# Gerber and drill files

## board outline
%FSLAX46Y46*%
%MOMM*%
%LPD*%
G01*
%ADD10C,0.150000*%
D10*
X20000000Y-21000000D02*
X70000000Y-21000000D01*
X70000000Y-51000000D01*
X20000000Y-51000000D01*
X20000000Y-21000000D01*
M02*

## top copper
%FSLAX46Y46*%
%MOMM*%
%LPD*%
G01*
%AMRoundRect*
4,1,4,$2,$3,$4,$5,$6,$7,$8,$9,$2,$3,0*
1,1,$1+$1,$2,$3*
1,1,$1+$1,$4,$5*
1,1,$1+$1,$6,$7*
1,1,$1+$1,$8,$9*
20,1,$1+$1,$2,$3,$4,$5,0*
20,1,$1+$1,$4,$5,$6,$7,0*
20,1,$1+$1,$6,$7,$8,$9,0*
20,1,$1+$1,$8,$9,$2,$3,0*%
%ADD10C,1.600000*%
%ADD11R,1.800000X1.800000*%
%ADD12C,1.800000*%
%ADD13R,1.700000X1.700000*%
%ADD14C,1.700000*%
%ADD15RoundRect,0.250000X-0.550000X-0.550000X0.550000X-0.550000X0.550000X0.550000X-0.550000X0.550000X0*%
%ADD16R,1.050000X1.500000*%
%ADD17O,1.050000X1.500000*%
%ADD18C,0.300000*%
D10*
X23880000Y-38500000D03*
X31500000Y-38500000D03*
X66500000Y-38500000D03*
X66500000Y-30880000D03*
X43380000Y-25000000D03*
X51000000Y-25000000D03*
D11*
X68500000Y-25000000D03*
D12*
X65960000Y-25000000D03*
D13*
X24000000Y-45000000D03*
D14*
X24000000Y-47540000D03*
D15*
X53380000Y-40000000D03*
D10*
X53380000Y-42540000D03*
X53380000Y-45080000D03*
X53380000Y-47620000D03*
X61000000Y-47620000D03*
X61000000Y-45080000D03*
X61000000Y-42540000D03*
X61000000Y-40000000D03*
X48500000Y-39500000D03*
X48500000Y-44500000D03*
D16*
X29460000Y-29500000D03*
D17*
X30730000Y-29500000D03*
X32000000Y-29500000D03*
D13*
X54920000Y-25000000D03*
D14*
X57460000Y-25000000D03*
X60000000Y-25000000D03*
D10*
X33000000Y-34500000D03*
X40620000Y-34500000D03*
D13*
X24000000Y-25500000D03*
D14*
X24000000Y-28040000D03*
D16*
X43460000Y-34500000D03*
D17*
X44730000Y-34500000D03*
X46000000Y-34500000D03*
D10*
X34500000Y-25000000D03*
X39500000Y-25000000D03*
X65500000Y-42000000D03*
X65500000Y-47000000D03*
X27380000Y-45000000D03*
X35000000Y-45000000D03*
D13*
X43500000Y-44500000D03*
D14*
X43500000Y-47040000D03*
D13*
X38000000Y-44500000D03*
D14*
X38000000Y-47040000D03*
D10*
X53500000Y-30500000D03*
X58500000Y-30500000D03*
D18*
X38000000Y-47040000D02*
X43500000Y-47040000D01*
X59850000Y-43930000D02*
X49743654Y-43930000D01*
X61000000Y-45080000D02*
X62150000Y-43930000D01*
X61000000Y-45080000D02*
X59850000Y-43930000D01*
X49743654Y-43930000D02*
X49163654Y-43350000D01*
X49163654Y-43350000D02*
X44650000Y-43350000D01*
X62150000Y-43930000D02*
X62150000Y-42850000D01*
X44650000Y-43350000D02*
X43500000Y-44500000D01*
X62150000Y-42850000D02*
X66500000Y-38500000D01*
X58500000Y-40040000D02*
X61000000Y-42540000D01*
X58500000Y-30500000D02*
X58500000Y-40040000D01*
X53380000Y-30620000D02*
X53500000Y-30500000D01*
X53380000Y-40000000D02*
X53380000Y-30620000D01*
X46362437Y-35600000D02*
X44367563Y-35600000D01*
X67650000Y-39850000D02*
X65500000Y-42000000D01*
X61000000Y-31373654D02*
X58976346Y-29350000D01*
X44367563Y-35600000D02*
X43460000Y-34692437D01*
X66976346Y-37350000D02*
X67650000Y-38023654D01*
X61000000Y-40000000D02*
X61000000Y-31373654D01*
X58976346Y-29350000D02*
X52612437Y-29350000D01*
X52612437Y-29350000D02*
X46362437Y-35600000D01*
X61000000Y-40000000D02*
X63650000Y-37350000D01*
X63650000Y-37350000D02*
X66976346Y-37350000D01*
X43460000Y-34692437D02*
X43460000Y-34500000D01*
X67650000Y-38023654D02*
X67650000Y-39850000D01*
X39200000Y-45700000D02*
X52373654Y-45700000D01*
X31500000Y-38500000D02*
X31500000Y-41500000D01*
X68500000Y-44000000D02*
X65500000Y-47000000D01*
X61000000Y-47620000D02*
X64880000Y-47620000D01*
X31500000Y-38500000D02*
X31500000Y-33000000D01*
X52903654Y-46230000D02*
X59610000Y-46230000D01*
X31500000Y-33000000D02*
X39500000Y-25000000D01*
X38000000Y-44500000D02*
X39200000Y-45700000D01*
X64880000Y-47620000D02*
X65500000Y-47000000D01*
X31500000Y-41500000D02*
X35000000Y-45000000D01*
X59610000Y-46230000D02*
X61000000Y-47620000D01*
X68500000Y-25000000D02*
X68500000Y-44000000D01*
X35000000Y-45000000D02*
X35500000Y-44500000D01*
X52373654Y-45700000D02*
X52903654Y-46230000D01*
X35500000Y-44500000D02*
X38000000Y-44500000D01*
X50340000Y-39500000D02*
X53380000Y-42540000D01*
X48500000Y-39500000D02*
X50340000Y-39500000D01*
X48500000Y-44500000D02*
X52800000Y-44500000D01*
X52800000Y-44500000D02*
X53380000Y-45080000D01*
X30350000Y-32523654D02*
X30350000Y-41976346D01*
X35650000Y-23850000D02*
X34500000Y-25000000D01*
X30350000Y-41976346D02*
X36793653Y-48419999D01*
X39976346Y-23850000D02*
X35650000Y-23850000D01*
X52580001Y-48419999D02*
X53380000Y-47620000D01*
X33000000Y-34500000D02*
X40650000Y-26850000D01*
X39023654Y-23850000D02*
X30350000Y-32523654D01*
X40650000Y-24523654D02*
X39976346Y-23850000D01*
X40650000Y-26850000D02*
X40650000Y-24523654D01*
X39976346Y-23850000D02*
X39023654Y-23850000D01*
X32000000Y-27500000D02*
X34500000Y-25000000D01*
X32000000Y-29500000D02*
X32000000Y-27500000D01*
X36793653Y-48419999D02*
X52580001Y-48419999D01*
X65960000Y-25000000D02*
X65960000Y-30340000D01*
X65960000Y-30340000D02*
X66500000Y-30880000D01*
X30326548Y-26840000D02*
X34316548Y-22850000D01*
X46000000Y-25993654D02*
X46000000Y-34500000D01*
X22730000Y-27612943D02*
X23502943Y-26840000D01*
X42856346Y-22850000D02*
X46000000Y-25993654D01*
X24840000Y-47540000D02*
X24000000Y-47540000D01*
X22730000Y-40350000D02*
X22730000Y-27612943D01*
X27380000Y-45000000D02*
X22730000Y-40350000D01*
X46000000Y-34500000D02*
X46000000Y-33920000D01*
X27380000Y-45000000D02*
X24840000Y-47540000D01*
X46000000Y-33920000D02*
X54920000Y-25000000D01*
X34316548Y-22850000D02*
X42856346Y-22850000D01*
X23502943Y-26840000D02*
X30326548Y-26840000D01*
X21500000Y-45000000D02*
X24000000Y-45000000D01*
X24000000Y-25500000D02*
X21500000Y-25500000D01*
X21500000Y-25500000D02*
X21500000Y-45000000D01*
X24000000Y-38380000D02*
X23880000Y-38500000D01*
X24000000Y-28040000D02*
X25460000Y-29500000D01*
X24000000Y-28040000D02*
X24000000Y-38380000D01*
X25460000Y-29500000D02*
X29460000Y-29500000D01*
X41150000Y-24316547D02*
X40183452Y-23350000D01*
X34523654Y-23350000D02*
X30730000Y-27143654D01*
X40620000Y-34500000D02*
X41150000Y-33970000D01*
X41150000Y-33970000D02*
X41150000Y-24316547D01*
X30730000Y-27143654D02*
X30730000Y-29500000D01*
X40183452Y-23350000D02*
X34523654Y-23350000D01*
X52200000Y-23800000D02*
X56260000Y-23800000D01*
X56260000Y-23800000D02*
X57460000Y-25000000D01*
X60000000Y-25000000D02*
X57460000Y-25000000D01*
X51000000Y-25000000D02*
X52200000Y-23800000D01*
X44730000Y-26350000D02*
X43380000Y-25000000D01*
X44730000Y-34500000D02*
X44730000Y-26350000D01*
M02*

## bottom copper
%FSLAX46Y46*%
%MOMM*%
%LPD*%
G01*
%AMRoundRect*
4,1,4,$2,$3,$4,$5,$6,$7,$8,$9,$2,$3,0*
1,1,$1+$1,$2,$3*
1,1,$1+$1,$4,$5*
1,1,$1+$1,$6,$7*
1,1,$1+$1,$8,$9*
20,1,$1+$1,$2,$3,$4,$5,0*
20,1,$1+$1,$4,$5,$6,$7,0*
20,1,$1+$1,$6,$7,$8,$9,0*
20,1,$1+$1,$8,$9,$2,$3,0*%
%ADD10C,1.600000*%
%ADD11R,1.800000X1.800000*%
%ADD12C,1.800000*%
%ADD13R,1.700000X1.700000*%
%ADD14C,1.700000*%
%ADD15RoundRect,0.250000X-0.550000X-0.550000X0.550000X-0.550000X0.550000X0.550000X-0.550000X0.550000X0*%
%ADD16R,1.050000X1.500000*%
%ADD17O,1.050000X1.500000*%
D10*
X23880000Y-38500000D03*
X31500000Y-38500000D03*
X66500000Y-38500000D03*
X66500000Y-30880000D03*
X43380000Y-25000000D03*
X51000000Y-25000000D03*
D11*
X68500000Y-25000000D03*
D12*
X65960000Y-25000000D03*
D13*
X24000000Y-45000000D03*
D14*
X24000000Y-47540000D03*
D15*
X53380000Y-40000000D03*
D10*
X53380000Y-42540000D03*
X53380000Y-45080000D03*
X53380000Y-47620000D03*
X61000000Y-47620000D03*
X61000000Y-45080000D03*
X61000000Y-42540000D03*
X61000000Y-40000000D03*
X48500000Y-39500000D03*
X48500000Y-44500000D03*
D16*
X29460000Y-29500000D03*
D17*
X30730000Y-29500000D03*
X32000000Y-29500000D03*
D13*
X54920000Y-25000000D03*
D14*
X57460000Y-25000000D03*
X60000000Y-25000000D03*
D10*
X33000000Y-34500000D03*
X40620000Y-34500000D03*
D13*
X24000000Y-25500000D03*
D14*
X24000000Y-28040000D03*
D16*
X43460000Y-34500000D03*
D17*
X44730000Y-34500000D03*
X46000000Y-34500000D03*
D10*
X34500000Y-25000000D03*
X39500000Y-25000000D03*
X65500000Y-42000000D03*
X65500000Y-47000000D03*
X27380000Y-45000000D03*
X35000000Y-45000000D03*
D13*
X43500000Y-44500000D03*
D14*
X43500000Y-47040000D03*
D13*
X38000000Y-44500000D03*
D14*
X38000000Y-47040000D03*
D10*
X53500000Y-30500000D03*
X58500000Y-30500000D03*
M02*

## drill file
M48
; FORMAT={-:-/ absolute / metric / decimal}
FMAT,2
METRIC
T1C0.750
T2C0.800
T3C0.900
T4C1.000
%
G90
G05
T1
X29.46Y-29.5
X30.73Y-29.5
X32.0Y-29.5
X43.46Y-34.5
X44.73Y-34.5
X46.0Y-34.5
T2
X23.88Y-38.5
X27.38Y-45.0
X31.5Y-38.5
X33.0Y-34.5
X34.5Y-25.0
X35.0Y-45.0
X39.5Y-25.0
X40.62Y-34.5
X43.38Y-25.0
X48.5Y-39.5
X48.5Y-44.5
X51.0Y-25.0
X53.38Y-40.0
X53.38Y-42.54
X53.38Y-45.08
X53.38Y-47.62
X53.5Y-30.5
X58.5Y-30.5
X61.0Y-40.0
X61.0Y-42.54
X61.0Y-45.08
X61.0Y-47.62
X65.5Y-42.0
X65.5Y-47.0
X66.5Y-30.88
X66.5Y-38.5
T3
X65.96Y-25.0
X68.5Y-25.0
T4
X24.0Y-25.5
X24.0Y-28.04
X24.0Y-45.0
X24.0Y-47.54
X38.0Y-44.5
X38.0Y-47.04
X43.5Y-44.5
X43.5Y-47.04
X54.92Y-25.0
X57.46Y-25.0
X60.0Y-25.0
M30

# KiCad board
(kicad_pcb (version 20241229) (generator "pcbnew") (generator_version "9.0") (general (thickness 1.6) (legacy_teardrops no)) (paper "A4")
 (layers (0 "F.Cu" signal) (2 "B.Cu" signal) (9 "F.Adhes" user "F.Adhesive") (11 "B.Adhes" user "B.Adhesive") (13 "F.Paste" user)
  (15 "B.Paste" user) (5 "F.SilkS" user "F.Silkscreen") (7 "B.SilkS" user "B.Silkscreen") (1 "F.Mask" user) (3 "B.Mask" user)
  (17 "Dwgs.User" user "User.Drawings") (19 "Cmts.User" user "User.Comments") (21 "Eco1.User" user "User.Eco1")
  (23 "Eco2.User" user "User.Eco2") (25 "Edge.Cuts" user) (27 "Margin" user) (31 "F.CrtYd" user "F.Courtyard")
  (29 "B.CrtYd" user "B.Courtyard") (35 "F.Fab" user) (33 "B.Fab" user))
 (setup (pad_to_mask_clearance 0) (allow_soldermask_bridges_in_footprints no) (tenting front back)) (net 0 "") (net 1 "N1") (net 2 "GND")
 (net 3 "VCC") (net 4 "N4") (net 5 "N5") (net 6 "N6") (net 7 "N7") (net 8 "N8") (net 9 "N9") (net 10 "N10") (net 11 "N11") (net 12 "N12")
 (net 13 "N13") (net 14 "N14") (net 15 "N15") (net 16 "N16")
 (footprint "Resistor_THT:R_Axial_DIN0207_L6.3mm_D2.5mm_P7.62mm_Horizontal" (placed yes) (layer "F.Cu") (at 23.88 38.5)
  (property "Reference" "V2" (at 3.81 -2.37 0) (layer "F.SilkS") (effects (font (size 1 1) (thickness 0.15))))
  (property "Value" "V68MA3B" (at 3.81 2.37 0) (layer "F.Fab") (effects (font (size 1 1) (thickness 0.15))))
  (pad "1" thru_hole circle (at 0 0) (size 1.6 1.6) (drill 0.8) (layers "*.Cu" "*.Mask") (remove_unused_layers no) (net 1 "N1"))
  (pad "2" thru_hole circle (at 7.62 0) (size 1.6 1.6) (drill 0.8) (layers "*.Cu" "*.Mask") (remove_unused_layers no) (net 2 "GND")))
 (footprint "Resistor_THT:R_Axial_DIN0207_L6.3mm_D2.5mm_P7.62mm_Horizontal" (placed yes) (layer "F.Cu") (at 66.5 38.5 90)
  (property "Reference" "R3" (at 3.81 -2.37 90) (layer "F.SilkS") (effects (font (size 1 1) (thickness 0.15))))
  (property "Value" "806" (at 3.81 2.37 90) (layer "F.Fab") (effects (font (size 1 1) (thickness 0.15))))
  (pad "1" thru_hole circle (at 0 0 90) (size 1.6 1.6) (drill 0.8) (layers "*.Cu" "*.Mask") (remove_unused_layers no) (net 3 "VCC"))
  (pad "2" thru_hole circle (at 7.62 0 90) (size 1.6 1.6) (drill 0.8) (layers "*.Cu" "*.Mask") (remove_unused_layers no) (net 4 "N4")))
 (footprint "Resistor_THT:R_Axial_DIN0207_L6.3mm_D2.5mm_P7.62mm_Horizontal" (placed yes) (layer "F.Cu") (at 43.38 25)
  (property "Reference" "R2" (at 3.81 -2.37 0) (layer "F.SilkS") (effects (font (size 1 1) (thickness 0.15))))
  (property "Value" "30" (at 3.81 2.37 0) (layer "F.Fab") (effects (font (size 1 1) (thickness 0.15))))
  (pad "1" thru_hole circle (at 0 0) (size 1.6 1.6) (drill 0.8) (layers "*.Cu" "*.Mask") (remove_unused_layers no) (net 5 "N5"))
  (pad "2" thru_hole circle (at 7.62 0) (size 1.6 1.6) (drill 0.8) (layers "*.Cu" "*.Mask") (remove_unused_layers no) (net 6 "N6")))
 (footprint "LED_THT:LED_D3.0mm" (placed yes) (layer "F.Cu") (at 68.5 25 180)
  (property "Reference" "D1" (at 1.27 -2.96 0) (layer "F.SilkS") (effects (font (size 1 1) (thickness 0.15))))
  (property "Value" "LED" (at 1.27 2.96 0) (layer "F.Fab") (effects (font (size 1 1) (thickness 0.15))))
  (pad "1" thru_hole rect (at 0 0 180) (size 1.8 1.8) (drill 0.9) (layers "*.Cu" "*.Mask") (remove_unused_layers no) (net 2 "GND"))
  (pad "2" thru_hole circle (at 2.54 0 180) (size 1.8 1.8) (drill 0.9) (layers "*.Cu" "*.Mask") (remove_unused_layers no) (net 4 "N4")))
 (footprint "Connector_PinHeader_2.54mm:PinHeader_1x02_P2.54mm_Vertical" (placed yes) (layer "F.Cu") (at 24 45)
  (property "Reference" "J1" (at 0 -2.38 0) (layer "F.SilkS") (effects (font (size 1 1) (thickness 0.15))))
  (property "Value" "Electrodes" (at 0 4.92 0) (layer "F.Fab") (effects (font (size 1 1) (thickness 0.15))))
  (pad "1" thru_hole rect (at 0 0) (size 1.7 1.7) (drill 1) (layers "*.Cu" "*.Mask") (remove_unused_layers no) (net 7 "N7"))
  (pad "2" thru_hole circle (at 0 2.54) (size 1.7 1.7) (drill 1) (layers "*.Cu" "*.Mask") (remove_unused_layers no) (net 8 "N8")))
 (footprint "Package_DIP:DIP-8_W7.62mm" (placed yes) (layer "F.Cu") (at 53.38 40)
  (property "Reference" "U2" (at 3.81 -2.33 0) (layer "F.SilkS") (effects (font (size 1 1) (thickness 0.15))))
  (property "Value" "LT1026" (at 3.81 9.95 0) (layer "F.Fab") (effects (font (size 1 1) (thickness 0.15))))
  (pad "1" thru_hole roundrect (at 0 0) (size 1.6 1.6) (drill 0.8) (layers "*.Cu" "*.Mask") (remove_unused_layers no)
   (roundrect_rratio 0.15625) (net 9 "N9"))
  (pad "2" thru_hole circle (at 0 2.54) (size 1.6 1.6) (drill 0.8) (layers "*.Cu" "*.Mask") (remove_unused_layers no) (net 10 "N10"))
  (pad "3" thru_hole circle (at 0 5.08) (size 1.6 1.6) (drill 0.8) (layers "*.Cu" "*.Mask") (remove_unused_layers no) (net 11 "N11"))
  (pad "4" thru_hole circle (at 0 7.62) (size 1.6 1.6) (drill 0.8) (layers "*.Cu" "*.Mask") (remove_unused_layers no) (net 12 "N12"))
  (pad "5" thru_hole circle (at 7.62 7.62) (size 1.6 1.6) (drill 0.8) (layers "*.Cu" "*.Mask") (remove_unused_layers no) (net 2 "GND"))
  (pad "6" thru_hole circle (at 7.62 5.08) (size 1.6 1.6) (drill 0.8) (layers "*.Cu" "*.Mask") (remove_unused_layers no) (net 3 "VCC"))
  (pad "7" thru_hole circle (at 7.62 2.54) (size 1.6 1.6) (drill 0.8) (layers "*.Cu" "*.Mask") (remove_unused_layers no) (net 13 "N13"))
  (pad "8" thru_hole circle (at 7.62 0) (size 1.6 1.6) (drill 0.8) (layers "*.Cu" "*.Mask") (remove_unused_layers no) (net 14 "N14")))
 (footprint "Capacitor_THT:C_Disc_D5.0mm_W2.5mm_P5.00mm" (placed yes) (layer "F.Cu") (at 48.5 39.5 -90)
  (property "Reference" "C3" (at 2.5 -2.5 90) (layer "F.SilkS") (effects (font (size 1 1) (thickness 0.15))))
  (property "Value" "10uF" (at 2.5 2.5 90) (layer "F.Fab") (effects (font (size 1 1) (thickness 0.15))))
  (pad "1" thru_hole circle (at 0 0 270) (size 1.6 1.6) (drill 0.8) (layers "*.Cu" "*.Mask") (remove_unused_layers no) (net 10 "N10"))
  (pad "2" thru_hole circle (at 5 0 270) (size 1.6 1.6) (drill 0.8) (layers "*.Cu" "*.Mask") (remove_unused_layers no) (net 11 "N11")))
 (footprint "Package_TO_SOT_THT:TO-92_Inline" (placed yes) (layer "F.Cu") (at 29.46 29.5)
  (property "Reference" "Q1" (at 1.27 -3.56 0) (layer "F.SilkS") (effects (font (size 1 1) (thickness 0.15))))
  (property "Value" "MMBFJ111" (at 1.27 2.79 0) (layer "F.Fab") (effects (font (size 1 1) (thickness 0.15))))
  (pad "1" thru_hole rect (at 0 0) (size 1.05 1.5) (drill 0.75) (layers "*.Cu" "*.Mask") (remove_unused_layers no) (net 1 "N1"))
  (pad "2" thru_hole oval (at 1.27 0) (size 1.05 1.5) (drill 0.75) (layers "*.Cu" "*.Mask") (remove_unused_layers no) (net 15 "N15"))
  (pad "3" thru_hole oval (at 2.54 0) (size 1.05 1.5) (drill 0.75) (layers "*.Cu" "*.Mask") (remove_unused_layers no) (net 12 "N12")))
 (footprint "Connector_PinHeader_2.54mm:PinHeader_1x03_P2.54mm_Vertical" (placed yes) (layer "F.Cu") (at 54.92 25 90)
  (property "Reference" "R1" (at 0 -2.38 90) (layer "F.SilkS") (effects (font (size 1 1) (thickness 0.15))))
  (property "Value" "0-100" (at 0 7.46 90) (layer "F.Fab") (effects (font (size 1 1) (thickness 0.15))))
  (pad "1" thru_hole rect (at 0 0 90) (size 1.7 1.7) (drill 1) (layers "*.Cu" "*.Mask") (remove_unused_layers no) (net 8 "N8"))
  (pad "2" thru_hole circle (at 0 2.54 90) (size 1.7 1.7) (drill 1) (layers "*.Cu" "*.Mask") (remove_unused_layers no) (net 6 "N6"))
  (pad "3" thru_hole circle (at 0 5.08 90) (size 1.7 1.7) (drill 1) (layers "*.Cu" "*.Mask") (remove_unused_layers no) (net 6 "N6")))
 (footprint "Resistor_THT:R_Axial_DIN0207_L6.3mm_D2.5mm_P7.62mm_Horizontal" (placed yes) (layer "F.Cu") (at 33 34.5)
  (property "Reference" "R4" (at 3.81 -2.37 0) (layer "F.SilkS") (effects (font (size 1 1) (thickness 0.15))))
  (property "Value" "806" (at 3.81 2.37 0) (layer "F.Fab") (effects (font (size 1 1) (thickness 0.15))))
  (pad "1" thru_hole circle (at 0 0) (size 1.6 1.6) (drill 0.8) (layers "*.Cu" "*.Mask") (remove_unused_layers no) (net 12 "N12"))
  (pad "2" thru_hole circle (at 7.62 0) (size 1.6 1.6) (drill 0.8) (layers "*.Cu" "*.Mask") (remove_unused_layers no) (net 15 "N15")))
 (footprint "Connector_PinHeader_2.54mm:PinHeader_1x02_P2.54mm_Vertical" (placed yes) (layer "F.Cu") (at 24 25.5)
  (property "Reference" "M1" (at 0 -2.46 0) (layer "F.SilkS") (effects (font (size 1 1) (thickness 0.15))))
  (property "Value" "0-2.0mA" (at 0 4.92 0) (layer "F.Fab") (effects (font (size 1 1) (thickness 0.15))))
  (pad "1" thru_hole rect (at 0 0) (size 1.7 1.7) (drill 1) (layers "*.Cu" "*.Mask") (remove_unused_layers no) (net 7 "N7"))
  (pad "2" thru_hole circle (at 0 2.54) (size 1.7 1.7) (drill 1) (layers "*.Cu" "*.Mask") (remove_unused_layers no) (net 1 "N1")))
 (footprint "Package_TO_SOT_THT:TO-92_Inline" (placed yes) (layer "F.Cu") (at 43.46 34.5)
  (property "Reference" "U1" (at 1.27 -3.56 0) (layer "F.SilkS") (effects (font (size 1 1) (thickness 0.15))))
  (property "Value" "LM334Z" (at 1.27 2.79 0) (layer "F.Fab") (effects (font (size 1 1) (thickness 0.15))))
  (pad "1" thru_hole rect (at 0 0) (size 1.05 1.5) (drill 0.75) (layers "*.Cu" "*.Mask") (remove_unused_layers no) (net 14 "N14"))
  (pad "2" thru_hole oval (at 1.27 0) (size 1.05 1.5) (drill 0.75) (layers "*.Cu" "*.Mask") (remove_unused_layers no) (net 5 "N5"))
  (pad "3" thru_hole oval (at 2.54 0) (size 1.05 1.5) (drill 0.75) (layers "*.Cu" "*.Mask") (remove_unused_layers no) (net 8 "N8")))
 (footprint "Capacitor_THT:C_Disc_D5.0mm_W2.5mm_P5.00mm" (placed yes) (layer "F.Cu") (at 34.5 25)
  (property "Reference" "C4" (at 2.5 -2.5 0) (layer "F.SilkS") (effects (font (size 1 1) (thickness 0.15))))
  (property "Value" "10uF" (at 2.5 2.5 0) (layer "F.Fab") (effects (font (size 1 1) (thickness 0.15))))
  (pad "1" thru_hole circle (at 0 0) (size 1.6 1.6) (drill 0.8) (layers "*.Cu" "*.Mask") (remove_unused_layers no) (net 12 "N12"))
  (pad "2" thru_hole circle (at 5 0) (size 1.6 1.6) (drill 0.8) (layers "*.Cu" "*.Mask") (remove_unused_layers no) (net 2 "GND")))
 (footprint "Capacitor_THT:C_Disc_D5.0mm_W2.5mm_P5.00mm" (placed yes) (layer "F.Cu") (at 65.5 42 -90)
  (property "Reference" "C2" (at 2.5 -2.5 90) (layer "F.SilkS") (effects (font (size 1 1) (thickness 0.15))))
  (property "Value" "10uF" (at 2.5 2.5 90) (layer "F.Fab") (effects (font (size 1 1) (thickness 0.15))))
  (pad "1" thru_hole circle (at 0 0 270) (size 1.6 1.6) (drill 0.8) (layers "*.Cu" "*.Mask") (remove_unused_layers no) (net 14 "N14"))
  (pad "2" thru_hole circle (at 5 0 270) (size 1.6 1.6) (drill 0.8) (layers "*.Cu" "*.Mask") (remove_unused_layers no) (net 2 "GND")))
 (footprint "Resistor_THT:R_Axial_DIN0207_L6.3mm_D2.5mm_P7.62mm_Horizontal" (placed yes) (layer "F.Cu") (at 27.38 45)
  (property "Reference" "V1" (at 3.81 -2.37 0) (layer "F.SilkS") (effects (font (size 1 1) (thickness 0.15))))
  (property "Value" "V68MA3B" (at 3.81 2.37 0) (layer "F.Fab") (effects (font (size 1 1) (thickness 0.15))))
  (pad "1" thru_hole circle (at 0 0) (size 1.6 1.6) (drill 0.8) (layers "*.Cu" "*.Mask") (remove_unused_layers no) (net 8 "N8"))
  (pad "2" thru_hole circle (at 7.62 0) (size 1.6 1.6) (drill 0.8) (layers "*.Cu" "*.Mask") (remove_unused_layers no) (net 2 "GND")))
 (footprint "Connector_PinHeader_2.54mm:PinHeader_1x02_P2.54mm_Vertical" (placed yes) (layer "F.Cu") (at 43.5 44.5)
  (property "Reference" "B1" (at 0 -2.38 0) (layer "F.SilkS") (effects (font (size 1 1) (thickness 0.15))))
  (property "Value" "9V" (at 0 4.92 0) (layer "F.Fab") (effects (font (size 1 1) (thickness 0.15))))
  (pad "1" thru_hole rect (at 0 0) (size 1.7 1.7) (drill 1) (layers "*.Cu" "*.Mask") (remove_unused_layers no) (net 3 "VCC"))
  (pad "2" thru_hole circle (at 0 2.54) (size 1.7 1.7) (drill 1) (layers "*.Cu" "*.Mask") (remove_unused_layers no) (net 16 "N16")))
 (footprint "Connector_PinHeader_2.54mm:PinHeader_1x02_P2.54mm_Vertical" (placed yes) (layer "F.Cu") (at 38 44.5)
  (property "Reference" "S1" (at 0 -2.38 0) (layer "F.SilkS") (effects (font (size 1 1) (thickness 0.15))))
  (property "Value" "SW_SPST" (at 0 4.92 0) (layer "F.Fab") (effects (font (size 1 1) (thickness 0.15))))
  (pad "1" thru_hole rect (at 0 0) (size 1.7 1.7) (drill 1) (layers "*.Cu" "*.Mask") (remove_unused_layers no) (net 2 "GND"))
  (pad "2" thru_hole circle (at 0 2.54) (size 1.7 1.7) (drill 1) (layers "*.Cu" "*.Mask") (remove_unused_layers no) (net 16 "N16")))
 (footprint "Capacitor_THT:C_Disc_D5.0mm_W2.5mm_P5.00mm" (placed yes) (layer "F.Cu") (at 53.5 30.5)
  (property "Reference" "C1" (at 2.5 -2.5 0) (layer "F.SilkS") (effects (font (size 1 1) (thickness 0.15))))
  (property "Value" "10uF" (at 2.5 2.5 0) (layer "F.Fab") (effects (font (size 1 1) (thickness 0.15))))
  (pad "1" thru_hole circle (at 0 0) (size 1.6 1.6) (drill 0.8) (layers "*.Cu" "*.Mask") (remove_unused_layers no) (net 9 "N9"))
  (pad "2" thru_hole circle (at 5 0) (size 1.6 1.6) (drill 0.8) (layers "*.Cu" "*.Mask") (remove_unused_layers no) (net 13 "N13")))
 (gr_rect (start 20 21) (end 70 51) (stroke (width 0.15) (type solid)) (fill no) (layer "Edge.Cuts"))
 (segment (start 38 47.04) (end 43.5 47.04) (width 0.3) (layer "F.Cu") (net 16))
 (segment (start 59.85 43.93) (end 49.743654 43.93) (width 0.3) (layer "F.Cu") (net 3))
 (segment (start 61 45.08) (end 62.15 43.93) (width 0.3) (layer "F.Cu") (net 3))
 (segment (start 61 45.08) (end 59.85 43.93) (width 0.3) (layer "F.Cu") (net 3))
 (segment (start 49.743654 43.93) (end 49.163654 43.35) (width 0.3) (layer "F.Cu") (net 3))
 (segment (start 49.163654 43.35) (end 44.65 43.35) (width 0.3) (layer "F.Cu") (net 3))
 (segment (start 62.15 43.93) (end 62.15 42.85) (width 0.3) (layer "F.Cu") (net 3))
 (segment (start 44.65 43.35) (end 43.5 44.5) (width 0.3) (layer "F.Cu") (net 3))
 (segment (start 62.15 42.85) (end 66.5 38.5) (width 0.3) (layer "F.Cu") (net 3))
 (segment (start 58.5 40.04) (end 61 42.54) (width 0.3) (layer "F.Cu") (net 13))
 (segment (start 58.5 30.5) (end 58.5 40.04) (width 0.3) (layer "F.Cu") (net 13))
 (segment (start 53.38 30.62) (end 53.5 30.5) (width 0.3) (layer "F.Cu") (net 9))
 (segment (start 53.38 40) (end 53.38 30.62) (width 0.3) (layer "F.Cu") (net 9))
 (segment (start 46.362437 35.6) (end 44.367563 35.6) (width 0.3) (layer "F.Cu") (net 14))
 (segment (start 67.65 39.85) (end 65.5 42) (width 0.3) (layer "F.Cu") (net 14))
 (segment (start 61 31.373654) (end 58.976346 29.35) (width 0.3) (layer "F.Cu") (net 14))
 (segment (start 44.367563 35.6) (end 43.46 34.692437) (width 0.3) (layer "F.Cu") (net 14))
 (segment (start 66.976346 37.35) (end 67.65 38.023654) (width 0.3) (layer "F.Cu") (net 14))
 (segment (start 61 40) (end 61 31.373654) (width 0.3) (layer "F.Cu") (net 14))
 (segment (start 58.976346 29.35) (end 52.612437 29.35) (width 0.3) (layer "F.Cu") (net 14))
 (segment (start 52.612437 29.35) (end 46.362437 35.6) (width 0.3) (layer "F.Cu") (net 14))
 (segment (start 61 40) (end 63.65 37.35) (width 0.3) (layer "F.Cu") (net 14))
 (segment (start 63.65 37.35) (end 66.976346 37.35) (width 0.3) (layer "F.Cu") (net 14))
 (segment (start 43.46 34.692437) (end 43.46 34.5) (width 0.3) (layer "F.Cu") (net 14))
 (segment (start 67.65 38.023654) (end 67.65 39.85) (width 0.3) (layer "F.Cu") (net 14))
 (segment (start 39.2 45.7) (end 52.373654 45.7) (width 0.3) (layer "F.Cu") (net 2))
 (segment (start 31.5 38.5) (end 31.5 41.5) (width 0.3) (layer "F.Cu") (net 2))
 (segment (start 68.5 44) (end 65.5 47) (width 0.3) (layer "F.Cu") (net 2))
 (segment (start 61 47.62) (end 64.88 47.62) (width 0.3) (layer "F.Cu") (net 2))
 (segment (start 31.5 38.5) (end 31.5 33) (width 0.3) (layer "F.Cu") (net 2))
 (segment (start 52.903654 46.23) (end 59.61 46.23) (width 0.3) (layer "F.Cu") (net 2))
 (segment (start 31.5 33) (end 39.5 25) (width 0.3) (layer "F.Cu") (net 2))
 (segment (start 38 44.5) (end 39.2 45.7) (width 0.3) (layer "F.Cu") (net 2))
 (segment (start 64.88 47.62) (end 65.5 47) (width 0.3) (layer "F.Cu") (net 2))
 (segment (start 31.5 41.5) (end 35 45) (width 0.3) (layer "F.Cu") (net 2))
 (segment (start 59.61 46.23) (end 61 47.62) (width 0.3) (layer "F.Cu") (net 2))
 (segment (start 68.5 25) (end 68.5 44) (width 0.3) (layer "F.Cu") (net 2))
 (segment (start 35 45) (end 35.5 44.5) (width 0.3) (layer "F.Cu") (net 2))
 (segment (start 52.373654 45.7) (end 52.903654 46.23) (width 0.3) (layer "F.Cu") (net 2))
 (segment (start 35.5 44.5) (end 38 44.5) (width 0.3) (layer "F.Cu") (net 2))
 (segment (start 50.34 39.5) (end 53.38 42.54) (width 0.3) (layer "F.Cu") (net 10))
 (segment (start 48.5 39.5) (end 50.34 39.5) (width 0.3) (layer "F.Cu") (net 10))
 (segment (start 48.5 44.5) (end 52.8 44.5) (width 0.3) (layer "F.Cu") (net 11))
 (segment (start 52.8 44.5) (end 53.38 45.08) (width 0.3) (layer "F.Cu") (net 11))
 (segment (start 30.35 32.523654) (end 30.35 41.976346) (width 0.3) (layer "F.Cu") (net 12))
 (segment (start 35.65 23.85) (end 34.5 25) (width 0.3) (layer "F.Cu") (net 12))
 (segment (start 30.35 41.976346) (end 36.793653 48.419999) (width 0.3) (layer "F.Cu") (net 12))
 (segment (start 39.976346 23.85) (end 35.65 23.85) (width 0.3) (layer "F.Cu") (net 12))
 (segment (start 52.580001 48.419999) (end 53.38 47.62) (width 0.3) (layer "F.Cu") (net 12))
 (segment (start 33 34.5) (end 40.65 26.85) (width 0.3) (layer "F.Cu") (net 12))
 (segment (start 39.023654 23.85) (end 30.35 32.523654) (width 0.3) (layer "F.Cu") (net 12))
 (segment (start 40.65 24.523654) (end 39.976346 23.85) (width 0.3) (layer "F.Cu") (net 12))
 (segment (start 40.65 26.85) (end 40.65 24.523654) (width 0.3) (layer "F.Cu") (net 12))
 (segment (start 39.976346 23.85) (end 39.023654 23.85) (width 0.3) (layer "F.Cu") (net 12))
 (segment (start 32 27.5) (end 34.5 25) (width 0.3) (layer "F.Cu") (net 12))
 (segment (start 32 29.5) (end 32 27.5) (width 0.3) (layer "F.Cu") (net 12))
 (segment (start 36.793653 48.419999) (end 52.580001 48.419999) (width 0.3) (layer "F.Cu") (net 12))
 (segment (start 65.96 25) (end 65.96 30.34) (width 0.3) (layer "F.Cu") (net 4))
 (segment (start 65.96 30.34) (end 66.5 30.88) (width 0.3) (layer "F.Cu") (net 4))
 (segment (start 30.326548 26.84) (end 34.316548 22.85) (width 0.3) (layer "F.Cu") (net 8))
 (segment (start 46 25.993654) (end 46 34.5) (width 0.3) (layer "F.Cu") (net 8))
 (segment (start 22.73 27.612943) (end 23.502943 26.84) (width 0.3) (layer "F.Cu") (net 8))
 (segment (start 42.856346 22.85) (end 46 25.993654) (width 0.3) (layer "F.Cu") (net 8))
 (segment (start 24.84 47.54) (end 24 47.54) (width 0.3) (layer "F.Cu") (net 8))
 (segment (start 22.73 40.35) (end 22.73 27.612943) (width 0.3) (layer "F.Cu") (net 8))
 (segment (start 27.38 45) (end 22.73 40.35) (width 0.3) (layer "F.Cu") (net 8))
 (segment (start 46 34.5) (end 46 33.92) (width 0.3) (layer "F.Cu") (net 8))
 (segment (start 27.38 45) (end 24.84 47.54) (width 0.3) (layer "F.Cu") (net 8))
 (segment (start 46 33.92) (end 54.92 25) (width 0.3) (layer "F.Cu") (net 8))
 (segment (start 34.316548 22.85) (end 42.856346 22.85) (width 0.3) (layer "F.Cu") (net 8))
 (segment (start 23.502943 26.84) (end 30.326548 26.84) (width 0.3) (layer "F.Cu") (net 8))
 (segment (start 21.5 45) (end 24 45) (width 0.3) (layer "F.Cu") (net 7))
 (segment (start 24 25.5) (end 21.5 25.5) (width 0.3) (layer "F.Cu") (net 7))
 (segment (start 21.5 25.5) (end 21.5 45) (width 0.3) (layer "F.Cu") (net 7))
 (segment (start 24 38.38) (end 23.88 38.5) (width 0.3) (layer "F.Cu") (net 1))
 (segment (start 24 28.04) (end 25.46 29.5) (width 0.3) (layer "F.Cu") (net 1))
 (segment (start 24 28.04) (end 24 38.38) (width 0.3) (layer "F.Cu") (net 1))
 (segment (start 25.46 29.5) (end 29.46 29.5) (width 0.3) (layer "F.Cu") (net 1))
 (segment (start 41.15 24.316547) (end 40.183452 23.35) (width 0.3) (layer "F.Cu") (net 15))
 (segment (start 34.523654 23.35) (end 30.73 27.143654) (width 0.3) (layer "F.Cu") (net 15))
 (segment (start 40.62 34.5) (end 41.15 33.97) (width 0.3) (layer "F.Cu") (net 15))
 (segment (start 41.15 33.97) (end 41.15 24.316547) (width 0.3) (layer "F.Cu") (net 15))
 (segment (start 30.73 27.143654) (end 30.73 29.5) (width 0.3) (layer "F.Cu") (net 15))
 (segment (start 40.183452 23.35) (end 34.523654 23.35) (width 0.3) (layer "F.Cu") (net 15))
 (segment (start 52.2 23.8) (end 56.26 23.8) (width 0.3) (layer "F.Cu") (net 6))
 (segment (start 56.26 23.8) (end 57.46 25) (width 0.3) (layer "F.Cu") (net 6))
 (segment (start 60 25) (end 57.46 25) (width 0.3) (layer "F.Cu") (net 6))
 (segment (start 51 25) (end 52.2 23.8) (width 0.3) (layer "F.Cu") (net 6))
 (segment (start 44.73 26.35) (end 43.38 25) (width 0.3) (layer "F.Cu") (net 5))
 (segment (start 44.73 34.5) (end 44.73 26.35) (width 0.3) (layer "F.Cu") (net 5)))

